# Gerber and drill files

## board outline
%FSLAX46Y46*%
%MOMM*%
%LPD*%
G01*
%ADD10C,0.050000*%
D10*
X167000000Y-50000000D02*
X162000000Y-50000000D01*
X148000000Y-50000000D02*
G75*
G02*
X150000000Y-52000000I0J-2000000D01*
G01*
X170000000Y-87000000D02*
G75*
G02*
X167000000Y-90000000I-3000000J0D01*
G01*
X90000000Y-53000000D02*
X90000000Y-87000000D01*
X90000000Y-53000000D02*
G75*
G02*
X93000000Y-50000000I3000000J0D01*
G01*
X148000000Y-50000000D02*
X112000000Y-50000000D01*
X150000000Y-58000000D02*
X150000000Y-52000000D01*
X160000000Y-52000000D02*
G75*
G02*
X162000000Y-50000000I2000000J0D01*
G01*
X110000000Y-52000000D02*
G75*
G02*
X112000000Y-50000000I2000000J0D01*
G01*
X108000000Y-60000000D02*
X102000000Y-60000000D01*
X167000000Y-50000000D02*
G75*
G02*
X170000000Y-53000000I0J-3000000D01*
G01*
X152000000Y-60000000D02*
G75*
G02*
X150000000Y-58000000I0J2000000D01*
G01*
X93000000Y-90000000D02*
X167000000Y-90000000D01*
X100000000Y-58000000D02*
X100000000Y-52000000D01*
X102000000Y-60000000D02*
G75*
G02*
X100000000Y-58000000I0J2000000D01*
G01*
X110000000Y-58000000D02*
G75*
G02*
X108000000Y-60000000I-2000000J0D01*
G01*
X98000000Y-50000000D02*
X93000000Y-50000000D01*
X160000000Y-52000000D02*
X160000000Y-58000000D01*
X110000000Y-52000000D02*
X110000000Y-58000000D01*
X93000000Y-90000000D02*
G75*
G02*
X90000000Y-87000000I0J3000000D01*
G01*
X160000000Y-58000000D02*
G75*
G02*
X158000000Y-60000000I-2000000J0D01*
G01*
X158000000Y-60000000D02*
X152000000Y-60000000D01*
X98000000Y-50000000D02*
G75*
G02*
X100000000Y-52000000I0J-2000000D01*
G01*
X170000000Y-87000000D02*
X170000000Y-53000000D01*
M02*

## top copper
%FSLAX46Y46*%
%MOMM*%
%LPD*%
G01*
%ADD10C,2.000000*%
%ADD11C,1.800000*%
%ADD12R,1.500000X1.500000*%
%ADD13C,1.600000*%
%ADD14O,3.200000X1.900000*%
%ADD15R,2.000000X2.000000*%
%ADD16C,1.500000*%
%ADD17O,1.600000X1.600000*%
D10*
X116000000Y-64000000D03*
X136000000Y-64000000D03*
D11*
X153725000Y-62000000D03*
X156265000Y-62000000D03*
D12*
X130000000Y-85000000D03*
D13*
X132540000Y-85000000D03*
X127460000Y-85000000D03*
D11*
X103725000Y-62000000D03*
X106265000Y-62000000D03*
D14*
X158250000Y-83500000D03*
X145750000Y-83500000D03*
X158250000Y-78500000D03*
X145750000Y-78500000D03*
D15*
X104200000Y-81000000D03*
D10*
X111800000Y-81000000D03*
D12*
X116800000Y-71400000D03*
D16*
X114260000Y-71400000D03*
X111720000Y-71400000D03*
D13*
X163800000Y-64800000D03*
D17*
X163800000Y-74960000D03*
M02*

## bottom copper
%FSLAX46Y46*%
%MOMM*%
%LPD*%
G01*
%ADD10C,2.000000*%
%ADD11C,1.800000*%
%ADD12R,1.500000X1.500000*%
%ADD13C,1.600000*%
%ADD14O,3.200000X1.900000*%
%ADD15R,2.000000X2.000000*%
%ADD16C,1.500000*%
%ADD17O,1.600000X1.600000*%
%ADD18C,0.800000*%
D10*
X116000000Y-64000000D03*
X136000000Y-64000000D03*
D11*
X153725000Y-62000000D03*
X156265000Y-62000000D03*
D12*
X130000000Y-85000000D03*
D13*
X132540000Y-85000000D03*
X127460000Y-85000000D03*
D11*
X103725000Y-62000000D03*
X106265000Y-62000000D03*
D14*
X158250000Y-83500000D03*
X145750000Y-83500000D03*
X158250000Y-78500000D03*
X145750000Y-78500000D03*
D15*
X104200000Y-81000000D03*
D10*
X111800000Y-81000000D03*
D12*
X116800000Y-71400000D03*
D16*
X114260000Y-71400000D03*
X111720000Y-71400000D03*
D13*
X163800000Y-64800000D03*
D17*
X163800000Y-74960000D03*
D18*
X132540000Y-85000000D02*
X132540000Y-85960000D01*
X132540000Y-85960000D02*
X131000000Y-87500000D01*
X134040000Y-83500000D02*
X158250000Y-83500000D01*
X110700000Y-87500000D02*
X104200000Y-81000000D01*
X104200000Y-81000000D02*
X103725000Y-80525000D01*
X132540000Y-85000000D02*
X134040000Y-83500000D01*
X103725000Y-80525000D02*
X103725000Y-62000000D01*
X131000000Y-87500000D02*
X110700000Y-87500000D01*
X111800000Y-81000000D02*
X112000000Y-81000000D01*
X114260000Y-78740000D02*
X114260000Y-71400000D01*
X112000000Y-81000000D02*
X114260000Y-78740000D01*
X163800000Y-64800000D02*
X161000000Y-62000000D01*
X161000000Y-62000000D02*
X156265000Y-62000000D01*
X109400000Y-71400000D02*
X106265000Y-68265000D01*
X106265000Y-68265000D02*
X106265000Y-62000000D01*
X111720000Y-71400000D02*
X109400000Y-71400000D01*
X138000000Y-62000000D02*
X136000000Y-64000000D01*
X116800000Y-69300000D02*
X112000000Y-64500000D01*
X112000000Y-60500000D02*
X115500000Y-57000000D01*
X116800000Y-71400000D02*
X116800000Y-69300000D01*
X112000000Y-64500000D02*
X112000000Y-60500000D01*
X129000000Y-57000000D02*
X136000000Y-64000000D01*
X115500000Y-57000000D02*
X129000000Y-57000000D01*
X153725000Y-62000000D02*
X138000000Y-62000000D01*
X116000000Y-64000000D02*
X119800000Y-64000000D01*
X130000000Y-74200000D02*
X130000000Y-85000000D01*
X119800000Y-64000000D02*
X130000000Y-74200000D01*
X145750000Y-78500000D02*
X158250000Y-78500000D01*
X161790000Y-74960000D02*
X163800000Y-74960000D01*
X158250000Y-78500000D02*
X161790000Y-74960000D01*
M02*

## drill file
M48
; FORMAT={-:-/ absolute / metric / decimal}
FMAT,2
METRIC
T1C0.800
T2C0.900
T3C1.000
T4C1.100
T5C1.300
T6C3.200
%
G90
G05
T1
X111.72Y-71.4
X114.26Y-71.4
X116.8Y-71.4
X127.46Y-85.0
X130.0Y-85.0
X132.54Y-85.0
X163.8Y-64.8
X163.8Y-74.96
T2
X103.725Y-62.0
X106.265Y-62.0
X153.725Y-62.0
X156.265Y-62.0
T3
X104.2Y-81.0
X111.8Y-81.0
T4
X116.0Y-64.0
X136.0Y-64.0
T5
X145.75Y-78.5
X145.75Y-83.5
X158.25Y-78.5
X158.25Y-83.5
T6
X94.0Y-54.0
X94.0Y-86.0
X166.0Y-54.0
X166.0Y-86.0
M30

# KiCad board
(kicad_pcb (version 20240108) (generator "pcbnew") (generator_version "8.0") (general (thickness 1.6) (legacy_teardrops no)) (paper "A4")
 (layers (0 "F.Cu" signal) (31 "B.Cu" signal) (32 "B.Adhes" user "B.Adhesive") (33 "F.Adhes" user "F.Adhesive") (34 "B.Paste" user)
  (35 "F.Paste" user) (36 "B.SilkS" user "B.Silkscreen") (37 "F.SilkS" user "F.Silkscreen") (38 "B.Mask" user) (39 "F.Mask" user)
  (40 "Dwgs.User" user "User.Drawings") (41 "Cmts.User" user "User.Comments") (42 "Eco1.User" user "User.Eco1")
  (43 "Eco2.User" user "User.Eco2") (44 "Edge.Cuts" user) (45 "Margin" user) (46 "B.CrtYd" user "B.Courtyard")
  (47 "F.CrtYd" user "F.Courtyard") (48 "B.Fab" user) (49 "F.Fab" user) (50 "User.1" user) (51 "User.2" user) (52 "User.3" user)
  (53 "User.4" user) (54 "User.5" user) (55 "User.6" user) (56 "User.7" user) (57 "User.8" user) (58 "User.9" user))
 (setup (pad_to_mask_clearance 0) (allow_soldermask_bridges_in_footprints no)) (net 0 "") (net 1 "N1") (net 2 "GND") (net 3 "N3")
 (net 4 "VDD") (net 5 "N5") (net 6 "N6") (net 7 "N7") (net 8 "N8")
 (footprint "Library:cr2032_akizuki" (layer "F.Cu") (at 130 64 -90)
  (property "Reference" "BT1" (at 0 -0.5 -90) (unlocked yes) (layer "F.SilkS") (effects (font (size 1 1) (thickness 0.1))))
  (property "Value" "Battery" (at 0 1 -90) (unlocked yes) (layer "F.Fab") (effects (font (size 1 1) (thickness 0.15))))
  (pad "1" thru_hole circle (at 0 14 270) (size 2 2) (drill 1.1) (layers "*.Cu" "*.Mask") (remove_unused_layers no) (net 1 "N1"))
  (pad "2" thru_hole circle (at 0 -6 270) (size 2 2) (drill 1.1) (layers "*.Cu" "*.Mask") (remove_unused_layers no) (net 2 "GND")))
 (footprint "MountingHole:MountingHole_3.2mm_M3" (layer "F.Cu") (at 94 54)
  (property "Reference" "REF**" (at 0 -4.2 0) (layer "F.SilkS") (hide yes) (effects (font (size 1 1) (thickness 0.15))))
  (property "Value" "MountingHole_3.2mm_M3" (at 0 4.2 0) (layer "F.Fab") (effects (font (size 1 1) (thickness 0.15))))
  (pad "" np_thru_hole circle (at 0 0) (size 3.2 3.2) (drill 3.2) (layers "F&B.Cu" "*.Mask")))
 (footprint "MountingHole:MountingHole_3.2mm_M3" (layer "F.Cu") (at 166 54)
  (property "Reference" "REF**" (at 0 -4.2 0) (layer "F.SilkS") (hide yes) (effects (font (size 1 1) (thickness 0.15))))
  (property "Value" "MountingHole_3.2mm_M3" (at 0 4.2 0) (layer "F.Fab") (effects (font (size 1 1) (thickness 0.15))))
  (pad "" np_thru_hole circle (at 0 0) (size 3.2 3.2) (drill 3.2) (layers "F&B.Cu" "*.Mask")))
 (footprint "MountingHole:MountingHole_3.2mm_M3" (layer "F.Cu") (at 94 86)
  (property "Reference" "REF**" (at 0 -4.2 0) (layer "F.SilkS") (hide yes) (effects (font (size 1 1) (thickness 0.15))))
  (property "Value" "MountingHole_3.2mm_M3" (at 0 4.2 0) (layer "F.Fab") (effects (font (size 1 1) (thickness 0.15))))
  (pad "" np_thru_hole circle (at 0 0) (size 3.2 3.2) (drill 3.2) (layers "*.Cu" "*.Mask")))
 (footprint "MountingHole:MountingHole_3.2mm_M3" (layer "F.Cu") (at 166 86)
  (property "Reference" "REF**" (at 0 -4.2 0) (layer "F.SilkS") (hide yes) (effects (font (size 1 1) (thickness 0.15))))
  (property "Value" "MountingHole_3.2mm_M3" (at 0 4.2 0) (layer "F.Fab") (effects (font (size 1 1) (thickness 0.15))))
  (pad "" np_thru_hole circle (at 0 0) (size 3.2 3.2) (drill 3.2) (layers "F&B.Cu" "*.Mask")))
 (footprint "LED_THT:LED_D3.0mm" (layer "F.Cu") (at 153.725 62)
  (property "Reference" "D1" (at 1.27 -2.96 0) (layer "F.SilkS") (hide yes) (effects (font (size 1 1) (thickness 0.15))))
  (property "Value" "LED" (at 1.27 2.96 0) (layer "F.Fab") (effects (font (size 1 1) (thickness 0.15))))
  (pad "1" thru_hole circle (at 0 0) (size 1.8 1.8) (drill 0.9) (layers "*.Cu" "*.Mask") (remove_unused_layers no) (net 2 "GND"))
  (pad "2" thru_hole circle (at 2.54 0) (size 1.8 1.8) (drill 0.9) (layers "*.Cu" "*.Mask") (remove_unused_layers no) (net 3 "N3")))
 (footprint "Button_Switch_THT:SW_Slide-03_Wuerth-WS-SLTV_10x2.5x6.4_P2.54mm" (layer "F.Cu") (at 130 85 180)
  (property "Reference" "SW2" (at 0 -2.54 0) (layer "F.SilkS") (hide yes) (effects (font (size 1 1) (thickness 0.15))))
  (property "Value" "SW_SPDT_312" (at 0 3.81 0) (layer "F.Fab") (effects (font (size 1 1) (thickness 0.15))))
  (pad "1" thru_hole rect (at 0 0 180) (size 1.5 1.5) (drill 0.8) (layers "*.Cu" "*.Mask") (remove_unused_layers no) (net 1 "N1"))
  (pad "2" thru_hole circle (at -2.54 0 180) (size 1.6 1.6) (drill 0.8) (layers "*.Cu" "*.Mask") (remove_unused_layers no) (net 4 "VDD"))
  (pad "3" thru_hole circle (at 2.54 0 180) (size 1.6 1.6) (drill 0.8) (layers "*.Cu" "*.Mask") (remove_unused_layers no) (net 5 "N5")))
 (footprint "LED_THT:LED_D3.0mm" (layer "F.Cu") (at 103.725 62)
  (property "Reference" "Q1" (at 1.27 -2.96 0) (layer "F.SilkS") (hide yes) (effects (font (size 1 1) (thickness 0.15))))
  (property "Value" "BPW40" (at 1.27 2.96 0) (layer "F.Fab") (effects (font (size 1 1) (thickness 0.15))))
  (pad "1" thru_hole circle (at 0 0) (size 1.8 1.8) (drill 0.9) (layers "*.Cu" "*.Mask") (remove_unused_layers no) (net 4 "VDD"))
  (pad "2" thru_hole circle (at 2.54 0) (size 1.8 1.8) (drill 0.9) (layers "*.Cu" "*.Mask") (remove_unused_layers no) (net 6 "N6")))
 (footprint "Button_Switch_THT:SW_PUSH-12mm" (layer "F.Cu") (at 158.25 83.5 180)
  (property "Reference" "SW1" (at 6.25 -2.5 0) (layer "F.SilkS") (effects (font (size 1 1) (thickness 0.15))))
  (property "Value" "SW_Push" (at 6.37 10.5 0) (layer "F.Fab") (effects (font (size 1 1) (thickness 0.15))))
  (pad "1" thru_hole oval (at 0 0 180) (size 3.2 1.9) (drill 1.3) (layers "*.Cu" "*.Mask") (remove_unused_layers no) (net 4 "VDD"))
  (pad "1" thru_hole oval (at 12.5 0 180) (size 3.2 1.9) (drill 1.3) (layers "*.Cu" "*.Mask") (remove_unused_layers no) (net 4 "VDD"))
  (pad "2" thru_hole oval (at 0 5 180) (size 3.2 1.9) (drill 1.3) (layers "*.Cu" "*.Mask") (remove_unused_layers no) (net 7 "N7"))
  (pad "2" thru_hole oval (at 12.5 5 180) (size 3.2 1.9) (drill 1.3) (layers "*.Cu" "*.Mask") (remove_unused_layers no) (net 7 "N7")))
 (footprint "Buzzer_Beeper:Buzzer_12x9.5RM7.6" (layer "F.Cu") (at 104.2 81)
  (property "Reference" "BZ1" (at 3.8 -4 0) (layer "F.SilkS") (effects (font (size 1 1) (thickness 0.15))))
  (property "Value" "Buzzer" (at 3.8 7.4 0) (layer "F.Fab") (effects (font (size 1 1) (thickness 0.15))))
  (pad "1" thru_hole rect (at 0 0) (size 2 2) (drill 1) (layers "*.Cu" "*.Mask") (remove_unused_layers no) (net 4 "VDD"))
  (pad "2" thru_hole circle (at 7.6 0) (size 2 2) (drill 1) (layers "*.Cu" "*.Mask") (remove_unused_layers no) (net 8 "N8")))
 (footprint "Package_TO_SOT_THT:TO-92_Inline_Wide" (layer "F.Cu") (at 116.8 71.4 180)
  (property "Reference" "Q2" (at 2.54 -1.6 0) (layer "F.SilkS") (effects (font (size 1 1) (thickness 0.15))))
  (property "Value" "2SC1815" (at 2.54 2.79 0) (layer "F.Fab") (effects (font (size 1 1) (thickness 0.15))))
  (pad "1" thru_hole rect (at 0 0 180) (size 1.5 1.5) (drill 0.8) (layers "*.Cu" "*.Mask") (remove_unused_layers no) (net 2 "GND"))
  (pad "2" thru_hole circle (at 2.54 0 180) (size 1.5 1.5) (drill 0.8) (layers "*.Cu" "*.Mask") (remove_unused_layers no) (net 8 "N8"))
  (pad "3" thru_hole circle (at 5.08 0 180) (size 1.5 1.5) (drill 0.8) (layers "*.Cu" "*.Mask") (remove_unused_layers no) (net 6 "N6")))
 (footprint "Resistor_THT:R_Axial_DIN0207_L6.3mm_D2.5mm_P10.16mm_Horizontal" (layer "F.Cu") (at 163.8 64.8 -90)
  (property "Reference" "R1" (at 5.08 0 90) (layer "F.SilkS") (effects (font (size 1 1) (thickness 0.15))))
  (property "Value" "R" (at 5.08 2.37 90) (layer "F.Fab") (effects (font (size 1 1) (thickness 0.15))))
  (pad "1" thru_hole circle (at 0 0 270) (size 1.6 1.6) (drill 0.8) (layers "*.Cu" "*.Mask") (remove_unused_layers no) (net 3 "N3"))
  (pad "2" thru_hole oval (at 10.16 0 270) (size 1.6 1.6) (drill 0.8) (layers "*.Cu" "*.Mask") (remove_unused_layers no) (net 7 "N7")))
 (gr_line (start 167 50) (end 162 50) (stroke (width 0.05) (type default)) (layer "Edge.Cuts"))
 (gr_arc (start 148 50) (mid 149.414214 50.585786) (end 150 52) (stroke (width 0.05) (type default)) (layer "Edge.Cuts"))
 (gr_arc (start 170 87) (mid 169.12132 89.12132) (end 167 90) (stroke (width 0.05) (type default)) (layer "Edge.Cuts"))
 (gr_line (start 90 53) (end 90 87) (stroke (width 0.05) (type default)) (layer "Edge.Cuts"))
 (gr_arc (start 90 53) (mid 90.87868 50.87868) (end 93 50) (stroke (width 0.05) (type default)) (layer "Edge.Cuts"))
 (gr_line (start 148 50) (end 112 50) (stroke (width 0.05) (type default)) (layer "Edge.Cuts"))
 (gr_line (start 150 58) (end 150 52) (stroke (width 0.05) (type default)) (layer "Edge.Cuts"))
 (gr_arc (start 160 52) (mid 160.585786 50.585786) (end 162 50) (stroke (width 0.05) (type default)) (layer "Edge.Cuts"))
 (gr_arc (start 110 52) (mid 110.585786 50.585786) (end 112 50) (stroke (width 0.05) (type default)) (layer "Edge.Cuts"))
 (gr_line (start 108 60) (end 102 60) (stroke (width 0.05) (type default)) (layer "Edge.Cuts"))
 (gr_arc (start 167 50) (mid 169.12132 50.87868) (end 170 53) (stroke (width 0.05) (type default)) (layer "Edge.Cuts"))
 (gr_arc (start 152 60) (mid 150.585786 59.414214) (end 150 58) (stroke (width 0.05) (type default)) (layer "Edge.Cuts"))
 (gr_line (start 93 90) (end 167 90) (stroke (width 0.05) (type default)) (layer "Edge.Cuts"))
 (gr_line (start 100 58) (end 100 52) (stroke (width 0.05) (type default)) (layer "Edge.Cuts"))
 (gr_arc (start 102 60) (mid 100.585786 59.414214) (end 100 58) (stroke (width 0.05) (type default)) (layer "Edge.Cuts"))
 (gr_arc (start 110 58) (mid 109.414214 59.414214) (end 108 60) (stroke (width 0.05) (type default)) (layer "Edge.Cuts"))
 (gr_line (start 98 50) (end 93 50) (stroke (width 0.05) (type default)) (layer "Edge.Cuts"))
 (gr_line (start 160 52) (end 160 58) (stroke (width 0.05) (type default)) (layer "Edge.Cuts"))
 (gr_line (start 110 52) (end 110 58) (stroke (width 0.05) (type default)) (layer "Edge.Cuts"))
 (gr_arc (start 93 90) (mid 90.87868 89.12132) (end 90 87) (stroke (width 0.05) (type default)) (layer "Edge.Cuts"))
 (gr_arc (start 160 58) (mid 159.414214 59.414214) (end 158 60) (stroke (width 0.05) (type default)) (layer "Edge.Cuts"))
 (gr_line (start 158 60) (end 152 60) (stroke (width 0.05) (type default)) (layer "Edge.Cuts"))
 (gr_arc (start 98 50) (mid 99.414214 50.585786) (end 100 52) (stroke (width 0.05) (type default)) (layer "Edge.Cuts"))
 (gr_line (start 170 87) (end 170 53) (stroke (width 0.05) (type default)) (layer "Edge.Cuts"))
 (segment (start 132.54 85) (end 132.54 85.96) (width 0.8) (layer "B.Cu") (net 4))
 (segment (start 132.54 85.96) (end 131 87.5) (width 0.8) (layer "B.Cu") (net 4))
 (segment (start 134.04 83.5) (end 158.25 83.5) (width 0.8) (layer "B.Cu") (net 4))
 (segment (start 110.7 87.5) (end 104.2 81) (width 0.8) (layer "B.Cu") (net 4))
 (segment (start 104.2 81) (end 103.725 80.525) (width 0.8) (layer "B.Cu") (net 4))
 (segment (start 132.54 85) (end 134.04 83.5) (width 0.8) (layer "B.Cu") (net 4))
 (segment (start 103.725 80.525) (end 103.725 62) (width 0.8) (layer "B.Cu") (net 4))
 (segment (start 131 87.5) (end 110.7 87.5) (width 0.8) (layer "B.Cu") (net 4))
 (segment (start 111.8 81) (end 112 81) (width 0.8) (layer "B.Cu") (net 8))
 (segment (start 114.26 78.74) (end 114.26 71.4) (width 0.8) (layer "B.Cu") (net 8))
 (segment (start 112 81) (end 114.26 78.74) (width 0.8) (layer "B.Cu") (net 8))
 (segment (start 163.8 64.8) (end 161 62) (width 0.8) (layer "B.Cu") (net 3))
 (segment (start 161 62) (end 156.265 62) (width 0.8) (layer "B.Cu") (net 3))
 (segment (start 109.4 71.4) (end 106.265 68.265) (width 0.8) (layer "B.Cu") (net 6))
 (segment (start 106.265 68.265) (end 106.265 62) (width 0.8) (layer "B.Cu") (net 6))
 (segment (start 111.72 71.4) (end 109.4 71.4) (width 0.8) (layer "B.Cu") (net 6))
 (segment (start 138 62) (end 136 64) (width 0.8) (layer "B.Cu") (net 2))
 (segment (start 116.8 69.3) (end 112 64.5) (width 0.8) (layer "B.Cu") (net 2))
 (segment (start 112 60.5) (end 115.5 57) (width 0.8) (layer "B.Cu") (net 2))
 (segment (start 116.8 71.4) (end 116.8 69.3) (width 0.8) (layer "B.Cu") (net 2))
 (segment (start 112 64.5) (end 112 60.5) (width 0.8) (layer "B.Cu") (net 2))
 (segment (start 129 57) (end 136 64) (width 0.8) (layer "B.Cu") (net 2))
 (segment (start 115.5 57) (end 129 57) (width 0.8) (layer "B.Cu") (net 2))
 (segment (start 153.725 62) (end 138 62) (width 0.8) (layer "B.Cu") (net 2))
 (segment (start 116 64) (end 119.8 64) (width 0.8) (layer "B.Cu") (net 1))
 (segment (start 130 74.2) (end 130 85) (width 0.8) (layer "B.Cu") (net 1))
 (segment (start 119.8 64) (end 130 74.2) (width 0.8) (layer "B.Cu") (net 1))
 (segment (start 145.75 78.5) (end 158.25 78.5) (width 0.8) (layer "B.Cu") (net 7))
 (segment (start 161.79 74.96) (end 163.8 74.96) (width 0.8) (layer "B.Cu") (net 7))
 (segment (start 158.25 78.5) (end 161.79 74.96) (width 0.8) (layer "B.Cu") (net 7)))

